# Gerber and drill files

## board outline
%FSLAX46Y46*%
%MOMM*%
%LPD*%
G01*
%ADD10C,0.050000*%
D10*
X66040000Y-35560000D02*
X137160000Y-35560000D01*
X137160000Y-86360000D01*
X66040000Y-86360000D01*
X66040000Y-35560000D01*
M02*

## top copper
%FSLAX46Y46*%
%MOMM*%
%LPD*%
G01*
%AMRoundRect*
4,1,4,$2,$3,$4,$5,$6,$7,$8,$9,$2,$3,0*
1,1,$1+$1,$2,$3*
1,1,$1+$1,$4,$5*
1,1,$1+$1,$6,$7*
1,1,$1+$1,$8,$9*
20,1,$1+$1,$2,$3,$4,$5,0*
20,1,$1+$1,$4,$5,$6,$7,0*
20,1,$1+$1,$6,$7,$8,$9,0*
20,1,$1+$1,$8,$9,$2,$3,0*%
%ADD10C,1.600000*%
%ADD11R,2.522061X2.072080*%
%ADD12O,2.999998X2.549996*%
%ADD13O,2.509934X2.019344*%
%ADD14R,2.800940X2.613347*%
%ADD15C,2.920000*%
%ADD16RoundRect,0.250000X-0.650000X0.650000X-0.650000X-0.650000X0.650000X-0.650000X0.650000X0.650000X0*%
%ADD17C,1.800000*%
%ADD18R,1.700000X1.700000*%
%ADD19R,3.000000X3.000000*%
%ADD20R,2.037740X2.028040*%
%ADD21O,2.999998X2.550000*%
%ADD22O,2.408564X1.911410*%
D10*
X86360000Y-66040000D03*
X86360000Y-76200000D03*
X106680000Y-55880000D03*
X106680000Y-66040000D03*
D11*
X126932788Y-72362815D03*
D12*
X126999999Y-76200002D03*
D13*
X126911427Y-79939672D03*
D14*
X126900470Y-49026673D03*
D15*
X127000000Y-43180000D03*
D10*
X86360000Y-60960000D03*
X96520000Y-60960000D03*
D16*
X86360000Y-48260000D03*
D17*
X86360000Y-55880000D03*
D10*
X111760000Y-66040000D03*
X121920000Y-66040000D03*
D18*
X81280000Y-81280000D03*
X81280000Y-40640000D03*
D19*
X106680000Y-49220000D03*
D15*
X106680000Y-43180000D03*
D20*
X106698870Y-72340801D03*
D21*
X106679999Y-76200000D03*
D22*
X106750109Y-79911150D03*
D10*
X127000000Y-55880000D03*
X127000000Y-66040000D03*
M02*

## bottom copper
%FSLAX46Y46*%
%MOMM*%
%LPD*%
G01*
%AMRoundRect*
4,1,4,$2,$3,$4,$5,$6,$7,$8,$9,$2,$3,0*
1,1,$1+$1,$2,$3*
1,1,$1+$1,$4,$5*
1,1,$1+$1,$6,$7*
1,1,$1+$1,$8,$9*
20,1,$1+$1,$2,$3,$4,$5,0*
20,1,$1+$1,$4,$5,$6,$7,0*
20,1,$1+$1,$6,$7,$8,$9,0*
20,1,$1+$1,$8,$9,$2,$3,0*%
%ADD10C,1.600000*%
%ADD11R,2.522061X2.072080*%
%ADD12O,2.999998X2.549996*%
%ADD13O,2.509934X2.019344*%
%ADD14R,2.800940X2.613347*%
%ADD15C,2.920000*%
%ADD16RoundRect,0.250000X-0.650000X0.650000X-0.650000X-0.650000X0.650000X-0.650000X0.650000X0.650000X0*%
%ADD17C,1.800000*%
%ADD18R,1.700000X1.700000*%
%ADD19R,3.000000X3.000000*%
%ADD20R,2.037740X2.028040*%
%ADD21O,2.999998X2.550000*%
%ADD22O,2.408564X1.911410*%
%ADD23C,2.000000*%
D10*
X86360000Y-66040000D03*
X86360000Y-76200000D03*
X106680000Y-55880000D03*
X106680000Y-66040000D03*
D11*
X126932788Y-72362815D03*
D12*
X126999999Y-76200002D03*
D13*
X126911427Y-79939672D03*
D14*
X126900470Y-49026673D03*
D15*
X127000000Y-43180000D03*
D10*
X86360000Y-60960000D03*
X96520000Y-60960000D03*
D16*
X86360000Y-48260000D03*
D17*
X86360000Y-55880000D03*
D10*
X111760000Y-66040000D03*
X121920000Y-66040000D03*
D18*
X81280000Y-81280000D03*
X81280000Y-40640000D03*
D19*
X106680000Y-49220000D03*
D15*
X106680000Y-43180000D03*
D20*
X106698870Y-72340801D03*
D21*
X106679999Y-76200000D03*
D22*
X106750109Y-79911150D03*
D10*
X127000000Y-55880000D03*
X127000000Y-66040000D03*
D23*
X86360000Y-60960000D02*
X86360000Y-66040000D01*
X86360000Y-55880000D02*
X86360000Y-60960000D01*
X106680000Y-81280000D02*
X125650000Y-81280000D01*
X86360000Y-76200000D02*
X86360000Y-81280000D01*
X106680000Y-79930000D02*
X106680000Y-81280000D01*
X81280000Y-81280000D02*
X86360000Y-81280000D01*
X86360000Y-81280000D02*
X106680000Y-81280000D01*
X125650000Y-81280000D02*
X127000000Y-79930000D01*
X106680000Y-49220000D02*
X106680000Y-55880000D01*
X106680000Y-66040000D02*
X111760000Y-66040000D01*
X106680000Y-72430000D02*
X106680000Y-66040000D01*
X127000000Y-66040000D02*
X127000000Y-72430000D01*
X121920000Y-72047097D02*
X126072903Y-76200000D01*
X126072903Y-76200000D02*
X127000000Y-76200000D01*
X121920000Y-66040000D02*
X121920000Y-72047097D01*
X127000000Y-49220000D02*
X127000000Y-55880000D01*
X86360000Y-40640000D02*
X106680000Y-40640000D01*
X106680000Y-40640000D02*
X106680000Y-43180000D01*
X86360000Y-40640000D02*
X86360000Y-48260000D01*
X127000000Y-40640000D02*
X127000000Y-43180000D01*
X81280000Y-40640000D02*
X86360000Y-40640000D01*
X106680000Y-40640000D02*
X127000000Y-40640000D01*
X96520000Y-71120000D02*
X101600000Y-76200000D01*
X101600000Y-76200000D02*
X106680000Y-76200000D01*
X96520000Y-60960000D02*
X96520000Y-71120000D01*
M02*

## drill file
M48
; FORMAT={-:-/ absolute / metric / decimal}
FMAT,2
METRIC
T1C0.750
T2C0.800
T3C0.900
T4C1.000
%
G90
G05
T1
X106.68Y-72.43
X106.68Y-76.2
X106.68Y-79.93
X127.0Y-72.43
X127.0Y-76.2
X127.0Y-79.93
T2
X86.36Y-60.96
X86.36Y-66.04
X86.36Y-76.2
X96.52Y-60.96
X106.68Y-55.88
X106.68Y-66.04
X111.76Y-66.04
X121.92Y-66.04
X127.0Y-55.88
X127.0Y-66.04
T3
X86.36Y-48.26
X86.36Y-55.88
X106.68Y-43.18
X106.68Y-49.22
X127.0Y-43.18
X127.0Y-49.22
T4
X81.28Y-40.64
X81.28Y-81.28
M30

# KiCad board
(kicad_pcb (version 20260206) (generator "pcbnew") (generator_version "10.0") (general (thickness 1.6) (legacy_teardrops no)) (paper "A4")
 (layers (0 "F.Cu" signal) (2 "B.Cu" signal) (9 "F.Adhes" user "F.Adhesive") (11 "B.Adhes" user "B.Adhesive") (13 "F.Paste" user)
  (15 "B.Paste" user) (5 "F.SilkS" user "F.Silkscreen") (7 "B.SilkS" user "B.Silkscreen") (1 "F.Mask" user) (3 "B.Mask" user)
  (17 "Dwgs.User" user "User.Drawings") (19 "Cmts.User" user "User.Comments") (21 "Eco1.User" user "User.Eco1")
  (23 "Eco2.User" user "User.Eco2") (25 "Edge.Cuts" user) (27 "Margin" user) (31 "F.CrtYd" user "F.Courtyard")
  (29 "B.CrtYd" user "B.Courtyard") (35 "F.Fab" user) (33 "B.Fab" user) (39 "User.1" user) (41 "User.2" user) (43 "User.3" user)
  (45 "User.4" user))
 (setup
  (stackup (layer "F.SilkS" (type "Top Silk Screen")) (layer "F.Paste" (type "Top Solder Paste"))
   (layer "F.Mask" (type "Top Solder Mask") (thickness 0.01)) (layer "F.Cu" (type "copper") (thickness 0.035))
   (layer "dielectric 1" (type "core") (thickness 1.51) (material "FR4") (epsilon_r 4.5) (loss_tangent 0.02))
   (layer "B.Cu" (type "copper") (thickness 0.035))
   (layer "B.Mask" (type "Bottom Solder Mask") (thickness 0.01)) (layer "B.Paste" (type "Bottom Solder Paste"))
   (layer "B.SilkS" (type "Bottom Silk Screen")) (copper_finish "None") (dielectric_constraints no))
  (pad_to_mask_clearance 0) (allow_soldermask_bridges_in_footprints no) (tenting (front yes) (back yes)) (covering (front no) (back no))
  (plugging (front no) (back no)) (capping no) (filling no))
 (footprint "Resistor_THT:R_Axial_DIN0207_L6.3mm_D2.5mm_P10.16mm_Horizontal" (layer "F.Cu") (at 86.36 66.04 -90)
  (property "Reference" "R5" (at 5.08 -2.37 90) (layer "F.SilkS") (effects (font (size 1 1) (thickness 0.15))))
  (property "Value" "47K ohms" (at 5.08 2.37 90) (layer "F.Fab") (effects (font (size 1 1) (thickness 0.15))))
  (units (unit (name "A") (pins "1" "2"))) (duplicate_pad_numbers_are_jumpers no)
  (pad "1" thru_hole circle (at 0 0 270) (size 1.6 1.6) (drill 0.8) (layers "*.Cu" "*.Mask") (remove_unused_layers no) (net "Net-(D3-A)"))
  (pad "2" thru_hole circle (at 10.16 0 270) (size 1.6 1.6) (drill 0.8) (layers "*.Cu" "*.Mask") (remove_unused_layers no) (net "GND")))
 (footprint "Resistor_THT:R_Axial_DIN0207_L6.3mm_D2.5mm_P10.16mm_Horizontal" (layer "F.Cu") (at 106.68 55.88 -90)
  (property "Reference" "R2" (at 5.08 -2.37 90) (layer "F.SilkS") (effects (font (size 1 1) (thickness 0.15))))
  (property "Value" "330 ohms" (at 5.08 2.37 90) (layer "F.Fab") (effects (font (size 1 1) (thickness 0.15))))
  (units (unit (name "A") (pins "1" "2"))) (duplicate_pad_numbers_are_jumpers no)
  (pad "1" thru_hole circle (at 0 0 270) (size 1.6 1.6) (drill 0.8) (layers "*.Cu" "*.Mask") (remove_unused_layers no) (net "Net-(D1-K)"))
  (pad "2" thru_hole circle (at 10.16 0 270) (size 1.6 1.6) (drill 0.8) (layers "*.Cu" "*.Mask") (remove_unused_layers no)
   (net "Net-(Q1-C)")))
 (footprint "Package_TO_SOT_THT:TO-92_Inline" (layer "F.Cu") (at 127 74.93 -90)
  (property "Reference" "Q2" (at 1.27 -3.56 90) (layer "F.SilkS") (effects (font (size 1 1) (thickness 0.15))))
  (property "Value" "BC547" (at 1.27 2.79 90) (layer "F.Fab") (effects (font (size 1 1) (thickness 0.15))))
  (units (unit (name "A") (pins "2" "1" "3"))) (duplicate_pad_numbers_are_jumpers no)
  (pad "1" thru_hole rect (at -2.5 0 270) (size 2.07208 2.522061) (drill 0.75 (offset -0.067185 0.067212)) (layers "*.Cu" "*.Mask")
   (remove_unused_layers no) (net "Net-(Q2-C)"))
  (pad "2" thru_hole oval (at 1.27 0 270) (size 2.549996 2.999998) (drill 0.75 (offset 0.000002 0.000001)) (layers "*.Cu" "*.Mask")
   (remove_unused_layers no) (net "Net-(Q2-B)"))
  (pad "3" thru_hole oval (at 5 0 270) (size 2.019344 2.509934) (drill 0.75 (offset 0.009672 0.088573)) (layers "*.Cu" "*.Mask")
   (remove_unused_layers no) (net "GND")))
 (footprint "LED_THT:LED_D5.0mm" (layer "F.Cu") (at 127 45.72 90)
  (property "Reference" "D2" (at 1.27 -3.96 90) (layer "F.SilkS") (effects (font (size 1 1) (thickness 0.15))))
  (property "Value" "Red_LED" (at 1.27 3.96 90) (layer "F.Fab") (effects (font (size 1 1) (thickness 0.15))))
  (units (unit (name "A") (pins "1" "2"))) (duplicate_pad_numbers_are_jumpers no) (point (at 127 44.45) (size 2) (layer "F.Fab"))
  (pad "1" thru_hole rect (at -3.5 0 90) (size 2.613347 2.80094) (drill 0.9 (offset 0.193327 -0.09953)) (layers "*.Cu" "*.Mask")
   (remove_unused_layers no) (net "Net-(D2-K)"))
  (pad "2" thru_hole circle (at 2.54 0 90) (size 2.92 2.92) (drill 0.9) (layers "*.Cu" "*.Mask") (remove_unused_layers no) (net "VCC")))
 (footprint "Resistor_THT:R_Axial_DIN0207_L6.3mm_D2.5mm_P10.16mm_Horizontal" (layer "F.Cu") (at 86.36 60.96)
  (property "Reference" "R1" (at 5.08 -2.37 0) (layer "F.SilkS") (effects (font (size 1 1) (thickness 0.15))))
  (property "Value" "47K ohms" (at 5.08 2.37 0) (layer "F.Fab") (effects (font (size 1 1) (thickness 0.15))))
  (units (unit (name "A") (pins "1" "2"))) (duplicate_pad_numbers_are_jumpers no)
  (pad "1" thru_hole circle (at 0 0) (size 1.6 1.6) (drill 0.8) (layers "*.Cu" "*.Mask") (remove_unused_layers no) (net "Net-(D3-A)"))
  (pad "2" thru_hole circle (at 10.16 0) (size 1.6 1.6) (drill 0.8) (layers "*.Cu" "*.Mask") (remove_unused_layers no) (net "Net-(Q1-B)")))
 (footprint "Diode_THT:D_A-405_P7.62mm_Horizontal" (layer "F.Cu") (at 86.36 48.26 -90)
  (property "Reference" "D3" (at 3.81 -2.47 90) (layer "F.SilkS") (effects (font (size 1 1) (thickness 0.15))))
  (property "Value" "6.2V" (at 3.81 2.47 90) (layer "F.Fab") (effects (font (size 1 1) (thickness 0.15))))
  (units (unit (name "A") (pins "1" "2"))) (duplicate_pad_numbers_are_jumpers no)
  (pad "1" thru_hole roundrect (at 0 0 270) (size 1.8 1.8) (drill 0.9) (layers "*.Cu" "*.Mask") (remove_unused_layers no)
   (roundrect_rratio 0.138889) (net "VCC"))
  (pad "2" thru_hole circle (at 7.62 0 270) (size 1.8 1.8) (drill 0.9) (layers "*.Cu" "*.Mask") (remove_unused_layers no) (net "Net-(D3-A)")))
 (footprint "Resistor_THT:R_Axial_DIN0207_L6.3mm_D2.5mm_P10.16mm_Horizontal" (layer "F.Cu") (at 111.76 66.04)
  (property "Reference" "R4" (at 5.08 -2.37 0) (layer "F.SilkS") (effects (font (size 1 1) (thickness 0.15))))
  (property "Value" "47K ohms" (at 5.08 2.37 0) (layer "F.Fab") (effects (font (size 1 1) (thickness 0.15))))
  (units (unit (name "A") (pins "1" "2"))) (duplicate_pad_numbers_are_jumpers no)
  (pad "1" thru_hole circle (at 0 0) (size 1.6 1.6) (drill 0.8) (layers "*.Cu" "*.Mask") (remove_unused_layers no) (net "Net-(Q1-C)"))
  (pad "2" thru_hole circle (at 10.16 0) (size 1.6 1.6) (drill 0.8) (layers "*.Cu" "*.Mask") (remove_unused_layers no) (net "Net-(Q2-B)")))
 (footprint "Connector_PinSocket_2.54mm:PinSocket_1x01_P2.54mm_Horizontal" (layer "F.Cu") (at 81.28 81.28)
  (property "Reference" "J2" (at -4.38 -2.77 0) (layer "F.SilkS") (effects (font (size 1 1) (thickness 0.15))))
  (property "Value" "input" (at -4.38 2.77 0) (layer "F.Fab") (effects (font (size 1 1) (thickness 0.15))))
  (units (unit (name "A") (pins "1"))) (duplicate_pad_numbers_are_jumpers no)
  (pad "1" thru_hole rect (at 0 0) (size 1.7 1.7) (drill 1) (layers "*.Cu" "*.Mask") (remove_unused_layers no) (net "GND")))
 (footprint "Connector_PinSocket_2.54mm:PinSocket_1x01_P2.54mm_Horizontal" (layer "F.Cu") (at 81.28 40.64)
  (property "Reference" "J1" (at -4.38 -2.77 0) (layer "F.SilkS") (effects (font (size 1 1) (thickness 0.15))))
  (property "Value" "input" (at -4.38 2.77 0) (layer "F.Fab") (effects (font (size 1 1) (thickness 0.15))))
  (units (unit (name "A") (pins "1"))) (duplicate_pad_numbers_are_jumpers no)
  (pad "1" thru_hole rect (at 0 0) (size 1.7 1.7) (drill 1) (layers "*.Cu" "*.Mask") (remove_unused_layers no) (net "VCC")))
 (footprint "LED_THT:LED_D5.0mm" (layer "F.Cu") (at 106.68 45.72 90)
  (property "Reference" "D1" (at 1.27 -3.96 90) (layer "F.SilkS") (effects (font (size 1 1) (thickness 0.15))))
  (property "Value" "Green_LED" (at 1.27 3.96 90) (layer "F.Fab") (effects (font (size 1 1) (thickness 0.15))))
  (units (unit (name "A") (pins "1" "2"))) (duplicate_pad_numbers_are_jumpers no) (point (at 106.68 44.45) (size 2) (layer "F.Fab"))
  (pad "1" thru_hole rect (at -3.5 0 90) (size 3 3) (drill 0.9) (layers "*.Cu" "*.Mask") (remove_unused_layers no) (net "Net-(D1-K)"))
  (pad "2" thru_hole circle (at 2.54 0 90) (size 2.92 2.92) (drill 0.9) (layers "*.Cu" "*.Mask") (remove_unused_layers no) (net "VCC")))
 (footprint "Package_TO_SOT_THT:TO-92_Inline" (layer "F.Cu") (at 106.68 74.93 -90)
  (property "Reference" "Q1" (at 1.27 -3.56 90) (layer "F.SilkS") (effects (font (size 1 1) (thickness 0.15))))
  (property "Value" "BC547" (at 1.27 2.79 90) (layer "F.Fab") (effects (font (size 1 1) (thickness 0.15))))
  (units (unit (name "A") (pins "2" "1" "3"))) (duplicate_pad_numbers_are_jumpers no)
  (pad "1" thru_hole rect (at -2.5 0 270) (size 2.02804 2.03774) (drill 0.75 (offset -0.089199 -0.01887)) (layers "*.Cu" "*.Mask")
   (remove_unused_layers no) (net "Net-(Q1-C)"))
  (pad "2" thru_hole oval (at 1.27 0 270) (size 2.55 2.999998) (drill 0.75 (offset 0 0.000001)) (layers "*.Cu" "*.Mask")
   (remove_unused_layers no) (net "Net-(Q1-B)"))
  (pad "3" thru_hole oval (at 5 0 270) (size 1.91141 2.408564) (drill 0.75 (offset -0.01885 -0.070109)) (layers "*.Cu" "*.Mask")
   (remove_unused_layers no) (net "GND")))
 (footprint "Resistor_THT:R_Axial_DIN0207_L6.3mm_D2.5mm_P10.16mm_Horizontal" (layer "F.Cu") (at 127 55.88 -90)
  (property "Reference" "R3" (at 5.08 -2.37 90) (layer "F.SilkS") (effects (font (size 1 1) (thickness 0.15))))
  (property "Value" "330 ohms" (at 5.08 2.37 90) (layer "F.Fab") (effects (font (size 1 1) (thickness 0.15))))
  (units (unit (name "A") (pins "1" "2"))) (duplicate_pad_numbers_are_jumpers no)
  (pad "1" thru_hole circle (at 0 0 270) (size 1.6 1.6) (drill 0.8) (layers "*.Cu" "*.Mask") (remove_unused_layers no) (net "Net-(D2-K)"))
  (pad "2" thru_hole circle (at 10.16 0 270) (size 1.6 1.6) (drill 0.8) (layers "*.Cu" "*.Mask") (remove_unused_layers no)
   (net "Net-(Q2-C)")))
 (gr_rect (start 66.04 35.56) (end 137.16 86.36) (stroke (width 0.05) (type default)) (fill no) (layer "Edge.Cuts"))
 (segment (start 86.36 60.96) (end 86.36 66.04) (width 2) (layer "B.Cu") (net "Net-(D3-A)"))
 (segment (start 86.36 55.88) (end 86.36 60.96) (width 2) (layer "B.Cu") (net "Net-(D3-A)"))
 (segment (start 106.68 81.28) (end 125.65 81.28) (width 2) (layer "B.Cu") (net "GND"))
 (segment (start 86.36 76.2) (end 86.36 81.28) (width 2) (layer "B.Cu") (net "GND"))
 (segment (start 106.68 79.93) (end 106.68 81.28) (width 2) (layer "B.Cu") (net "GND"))
 (segment (start 81.28 81.28) (end 86.36 81.28) (width 2) (layer "B.Cu") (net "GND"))
 (segment (start 86.36 81.28) (end 106.68 81.28) (width 2) (layer "B.Cu") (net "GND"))
 (segment (start 125.65 81.28) (end 127 79.93) (width 2) (layer "B.Cu") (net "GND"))
 (segment (start 106.68 49.22) (end 106.68 55.88) (width 2) (layer "B.Cu") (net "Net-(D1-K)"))
 (segment (start 106.68 66.04) (end 111.76 66.04) (width 2) (layer "B.Cu") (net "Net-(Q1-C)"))
 (segment (start 106.68 72.43) (end 106.68 66.04) (width 2) (layer "B.Cu") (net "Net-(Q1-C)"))
 (segment (start 127 66.04) (end 127 72.43) (width 2) (layer "B.Cu") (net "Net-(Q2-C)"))
 (segment (start 121.92 72.047097) (end 126.072903 76.2) (width 2) (layer "B.Cu") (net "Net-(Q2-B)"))
 (segment (start 126.072903 76.2) (end 127 76.2) (width 2) (layer "B.Cu") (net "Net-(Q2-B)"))
 (segment (start 121.92 66.04) (end 121.92 72.047097) (width 2) (layer "B.Cu") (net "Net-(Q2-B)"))
 (segment (start 127 49.22) (end 127 55.88) (width 2) (layer "B.Cu") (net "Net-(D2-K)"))
 (segment (start 86.36 40.64) (end 106.68 40.64) (width 2) (layer "B.Cu") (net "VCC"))
 (segment (start 106.68 40.64) (end 106.68 43.18) (width 2) (layer "B.Cu") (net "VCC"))
 (segment (start 86.36 40.64) (end 86.36 48.26) (width 2) (layer "B.Cu") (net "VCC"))
 (segment (start 127 40.64) (end 127 43.18) (width 2) (layer "B.Cu") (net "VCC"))
 (segment (start 81.28 40.64) (end 86.36 40.64) (width 2) (layer "B.Cu") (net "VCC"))
 (segment (start 106.68 40.64) (end 127 40.64) (width 2) (layer "B.Cu") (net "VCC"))
 (segment (start 96.52 71.12) (end 101.6 76.2) (width 2) (layer "B.Cu") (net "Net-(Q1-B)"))
 (segment (start 101.6 76.2) (end 106.68 76.2) (width 2) (layer "B.Cu") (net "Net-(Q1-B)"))
 (segment (start 96.52 60.96) (end 96.52 71.12) (width 2) (layer "B.Cu") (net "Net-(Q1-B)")))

